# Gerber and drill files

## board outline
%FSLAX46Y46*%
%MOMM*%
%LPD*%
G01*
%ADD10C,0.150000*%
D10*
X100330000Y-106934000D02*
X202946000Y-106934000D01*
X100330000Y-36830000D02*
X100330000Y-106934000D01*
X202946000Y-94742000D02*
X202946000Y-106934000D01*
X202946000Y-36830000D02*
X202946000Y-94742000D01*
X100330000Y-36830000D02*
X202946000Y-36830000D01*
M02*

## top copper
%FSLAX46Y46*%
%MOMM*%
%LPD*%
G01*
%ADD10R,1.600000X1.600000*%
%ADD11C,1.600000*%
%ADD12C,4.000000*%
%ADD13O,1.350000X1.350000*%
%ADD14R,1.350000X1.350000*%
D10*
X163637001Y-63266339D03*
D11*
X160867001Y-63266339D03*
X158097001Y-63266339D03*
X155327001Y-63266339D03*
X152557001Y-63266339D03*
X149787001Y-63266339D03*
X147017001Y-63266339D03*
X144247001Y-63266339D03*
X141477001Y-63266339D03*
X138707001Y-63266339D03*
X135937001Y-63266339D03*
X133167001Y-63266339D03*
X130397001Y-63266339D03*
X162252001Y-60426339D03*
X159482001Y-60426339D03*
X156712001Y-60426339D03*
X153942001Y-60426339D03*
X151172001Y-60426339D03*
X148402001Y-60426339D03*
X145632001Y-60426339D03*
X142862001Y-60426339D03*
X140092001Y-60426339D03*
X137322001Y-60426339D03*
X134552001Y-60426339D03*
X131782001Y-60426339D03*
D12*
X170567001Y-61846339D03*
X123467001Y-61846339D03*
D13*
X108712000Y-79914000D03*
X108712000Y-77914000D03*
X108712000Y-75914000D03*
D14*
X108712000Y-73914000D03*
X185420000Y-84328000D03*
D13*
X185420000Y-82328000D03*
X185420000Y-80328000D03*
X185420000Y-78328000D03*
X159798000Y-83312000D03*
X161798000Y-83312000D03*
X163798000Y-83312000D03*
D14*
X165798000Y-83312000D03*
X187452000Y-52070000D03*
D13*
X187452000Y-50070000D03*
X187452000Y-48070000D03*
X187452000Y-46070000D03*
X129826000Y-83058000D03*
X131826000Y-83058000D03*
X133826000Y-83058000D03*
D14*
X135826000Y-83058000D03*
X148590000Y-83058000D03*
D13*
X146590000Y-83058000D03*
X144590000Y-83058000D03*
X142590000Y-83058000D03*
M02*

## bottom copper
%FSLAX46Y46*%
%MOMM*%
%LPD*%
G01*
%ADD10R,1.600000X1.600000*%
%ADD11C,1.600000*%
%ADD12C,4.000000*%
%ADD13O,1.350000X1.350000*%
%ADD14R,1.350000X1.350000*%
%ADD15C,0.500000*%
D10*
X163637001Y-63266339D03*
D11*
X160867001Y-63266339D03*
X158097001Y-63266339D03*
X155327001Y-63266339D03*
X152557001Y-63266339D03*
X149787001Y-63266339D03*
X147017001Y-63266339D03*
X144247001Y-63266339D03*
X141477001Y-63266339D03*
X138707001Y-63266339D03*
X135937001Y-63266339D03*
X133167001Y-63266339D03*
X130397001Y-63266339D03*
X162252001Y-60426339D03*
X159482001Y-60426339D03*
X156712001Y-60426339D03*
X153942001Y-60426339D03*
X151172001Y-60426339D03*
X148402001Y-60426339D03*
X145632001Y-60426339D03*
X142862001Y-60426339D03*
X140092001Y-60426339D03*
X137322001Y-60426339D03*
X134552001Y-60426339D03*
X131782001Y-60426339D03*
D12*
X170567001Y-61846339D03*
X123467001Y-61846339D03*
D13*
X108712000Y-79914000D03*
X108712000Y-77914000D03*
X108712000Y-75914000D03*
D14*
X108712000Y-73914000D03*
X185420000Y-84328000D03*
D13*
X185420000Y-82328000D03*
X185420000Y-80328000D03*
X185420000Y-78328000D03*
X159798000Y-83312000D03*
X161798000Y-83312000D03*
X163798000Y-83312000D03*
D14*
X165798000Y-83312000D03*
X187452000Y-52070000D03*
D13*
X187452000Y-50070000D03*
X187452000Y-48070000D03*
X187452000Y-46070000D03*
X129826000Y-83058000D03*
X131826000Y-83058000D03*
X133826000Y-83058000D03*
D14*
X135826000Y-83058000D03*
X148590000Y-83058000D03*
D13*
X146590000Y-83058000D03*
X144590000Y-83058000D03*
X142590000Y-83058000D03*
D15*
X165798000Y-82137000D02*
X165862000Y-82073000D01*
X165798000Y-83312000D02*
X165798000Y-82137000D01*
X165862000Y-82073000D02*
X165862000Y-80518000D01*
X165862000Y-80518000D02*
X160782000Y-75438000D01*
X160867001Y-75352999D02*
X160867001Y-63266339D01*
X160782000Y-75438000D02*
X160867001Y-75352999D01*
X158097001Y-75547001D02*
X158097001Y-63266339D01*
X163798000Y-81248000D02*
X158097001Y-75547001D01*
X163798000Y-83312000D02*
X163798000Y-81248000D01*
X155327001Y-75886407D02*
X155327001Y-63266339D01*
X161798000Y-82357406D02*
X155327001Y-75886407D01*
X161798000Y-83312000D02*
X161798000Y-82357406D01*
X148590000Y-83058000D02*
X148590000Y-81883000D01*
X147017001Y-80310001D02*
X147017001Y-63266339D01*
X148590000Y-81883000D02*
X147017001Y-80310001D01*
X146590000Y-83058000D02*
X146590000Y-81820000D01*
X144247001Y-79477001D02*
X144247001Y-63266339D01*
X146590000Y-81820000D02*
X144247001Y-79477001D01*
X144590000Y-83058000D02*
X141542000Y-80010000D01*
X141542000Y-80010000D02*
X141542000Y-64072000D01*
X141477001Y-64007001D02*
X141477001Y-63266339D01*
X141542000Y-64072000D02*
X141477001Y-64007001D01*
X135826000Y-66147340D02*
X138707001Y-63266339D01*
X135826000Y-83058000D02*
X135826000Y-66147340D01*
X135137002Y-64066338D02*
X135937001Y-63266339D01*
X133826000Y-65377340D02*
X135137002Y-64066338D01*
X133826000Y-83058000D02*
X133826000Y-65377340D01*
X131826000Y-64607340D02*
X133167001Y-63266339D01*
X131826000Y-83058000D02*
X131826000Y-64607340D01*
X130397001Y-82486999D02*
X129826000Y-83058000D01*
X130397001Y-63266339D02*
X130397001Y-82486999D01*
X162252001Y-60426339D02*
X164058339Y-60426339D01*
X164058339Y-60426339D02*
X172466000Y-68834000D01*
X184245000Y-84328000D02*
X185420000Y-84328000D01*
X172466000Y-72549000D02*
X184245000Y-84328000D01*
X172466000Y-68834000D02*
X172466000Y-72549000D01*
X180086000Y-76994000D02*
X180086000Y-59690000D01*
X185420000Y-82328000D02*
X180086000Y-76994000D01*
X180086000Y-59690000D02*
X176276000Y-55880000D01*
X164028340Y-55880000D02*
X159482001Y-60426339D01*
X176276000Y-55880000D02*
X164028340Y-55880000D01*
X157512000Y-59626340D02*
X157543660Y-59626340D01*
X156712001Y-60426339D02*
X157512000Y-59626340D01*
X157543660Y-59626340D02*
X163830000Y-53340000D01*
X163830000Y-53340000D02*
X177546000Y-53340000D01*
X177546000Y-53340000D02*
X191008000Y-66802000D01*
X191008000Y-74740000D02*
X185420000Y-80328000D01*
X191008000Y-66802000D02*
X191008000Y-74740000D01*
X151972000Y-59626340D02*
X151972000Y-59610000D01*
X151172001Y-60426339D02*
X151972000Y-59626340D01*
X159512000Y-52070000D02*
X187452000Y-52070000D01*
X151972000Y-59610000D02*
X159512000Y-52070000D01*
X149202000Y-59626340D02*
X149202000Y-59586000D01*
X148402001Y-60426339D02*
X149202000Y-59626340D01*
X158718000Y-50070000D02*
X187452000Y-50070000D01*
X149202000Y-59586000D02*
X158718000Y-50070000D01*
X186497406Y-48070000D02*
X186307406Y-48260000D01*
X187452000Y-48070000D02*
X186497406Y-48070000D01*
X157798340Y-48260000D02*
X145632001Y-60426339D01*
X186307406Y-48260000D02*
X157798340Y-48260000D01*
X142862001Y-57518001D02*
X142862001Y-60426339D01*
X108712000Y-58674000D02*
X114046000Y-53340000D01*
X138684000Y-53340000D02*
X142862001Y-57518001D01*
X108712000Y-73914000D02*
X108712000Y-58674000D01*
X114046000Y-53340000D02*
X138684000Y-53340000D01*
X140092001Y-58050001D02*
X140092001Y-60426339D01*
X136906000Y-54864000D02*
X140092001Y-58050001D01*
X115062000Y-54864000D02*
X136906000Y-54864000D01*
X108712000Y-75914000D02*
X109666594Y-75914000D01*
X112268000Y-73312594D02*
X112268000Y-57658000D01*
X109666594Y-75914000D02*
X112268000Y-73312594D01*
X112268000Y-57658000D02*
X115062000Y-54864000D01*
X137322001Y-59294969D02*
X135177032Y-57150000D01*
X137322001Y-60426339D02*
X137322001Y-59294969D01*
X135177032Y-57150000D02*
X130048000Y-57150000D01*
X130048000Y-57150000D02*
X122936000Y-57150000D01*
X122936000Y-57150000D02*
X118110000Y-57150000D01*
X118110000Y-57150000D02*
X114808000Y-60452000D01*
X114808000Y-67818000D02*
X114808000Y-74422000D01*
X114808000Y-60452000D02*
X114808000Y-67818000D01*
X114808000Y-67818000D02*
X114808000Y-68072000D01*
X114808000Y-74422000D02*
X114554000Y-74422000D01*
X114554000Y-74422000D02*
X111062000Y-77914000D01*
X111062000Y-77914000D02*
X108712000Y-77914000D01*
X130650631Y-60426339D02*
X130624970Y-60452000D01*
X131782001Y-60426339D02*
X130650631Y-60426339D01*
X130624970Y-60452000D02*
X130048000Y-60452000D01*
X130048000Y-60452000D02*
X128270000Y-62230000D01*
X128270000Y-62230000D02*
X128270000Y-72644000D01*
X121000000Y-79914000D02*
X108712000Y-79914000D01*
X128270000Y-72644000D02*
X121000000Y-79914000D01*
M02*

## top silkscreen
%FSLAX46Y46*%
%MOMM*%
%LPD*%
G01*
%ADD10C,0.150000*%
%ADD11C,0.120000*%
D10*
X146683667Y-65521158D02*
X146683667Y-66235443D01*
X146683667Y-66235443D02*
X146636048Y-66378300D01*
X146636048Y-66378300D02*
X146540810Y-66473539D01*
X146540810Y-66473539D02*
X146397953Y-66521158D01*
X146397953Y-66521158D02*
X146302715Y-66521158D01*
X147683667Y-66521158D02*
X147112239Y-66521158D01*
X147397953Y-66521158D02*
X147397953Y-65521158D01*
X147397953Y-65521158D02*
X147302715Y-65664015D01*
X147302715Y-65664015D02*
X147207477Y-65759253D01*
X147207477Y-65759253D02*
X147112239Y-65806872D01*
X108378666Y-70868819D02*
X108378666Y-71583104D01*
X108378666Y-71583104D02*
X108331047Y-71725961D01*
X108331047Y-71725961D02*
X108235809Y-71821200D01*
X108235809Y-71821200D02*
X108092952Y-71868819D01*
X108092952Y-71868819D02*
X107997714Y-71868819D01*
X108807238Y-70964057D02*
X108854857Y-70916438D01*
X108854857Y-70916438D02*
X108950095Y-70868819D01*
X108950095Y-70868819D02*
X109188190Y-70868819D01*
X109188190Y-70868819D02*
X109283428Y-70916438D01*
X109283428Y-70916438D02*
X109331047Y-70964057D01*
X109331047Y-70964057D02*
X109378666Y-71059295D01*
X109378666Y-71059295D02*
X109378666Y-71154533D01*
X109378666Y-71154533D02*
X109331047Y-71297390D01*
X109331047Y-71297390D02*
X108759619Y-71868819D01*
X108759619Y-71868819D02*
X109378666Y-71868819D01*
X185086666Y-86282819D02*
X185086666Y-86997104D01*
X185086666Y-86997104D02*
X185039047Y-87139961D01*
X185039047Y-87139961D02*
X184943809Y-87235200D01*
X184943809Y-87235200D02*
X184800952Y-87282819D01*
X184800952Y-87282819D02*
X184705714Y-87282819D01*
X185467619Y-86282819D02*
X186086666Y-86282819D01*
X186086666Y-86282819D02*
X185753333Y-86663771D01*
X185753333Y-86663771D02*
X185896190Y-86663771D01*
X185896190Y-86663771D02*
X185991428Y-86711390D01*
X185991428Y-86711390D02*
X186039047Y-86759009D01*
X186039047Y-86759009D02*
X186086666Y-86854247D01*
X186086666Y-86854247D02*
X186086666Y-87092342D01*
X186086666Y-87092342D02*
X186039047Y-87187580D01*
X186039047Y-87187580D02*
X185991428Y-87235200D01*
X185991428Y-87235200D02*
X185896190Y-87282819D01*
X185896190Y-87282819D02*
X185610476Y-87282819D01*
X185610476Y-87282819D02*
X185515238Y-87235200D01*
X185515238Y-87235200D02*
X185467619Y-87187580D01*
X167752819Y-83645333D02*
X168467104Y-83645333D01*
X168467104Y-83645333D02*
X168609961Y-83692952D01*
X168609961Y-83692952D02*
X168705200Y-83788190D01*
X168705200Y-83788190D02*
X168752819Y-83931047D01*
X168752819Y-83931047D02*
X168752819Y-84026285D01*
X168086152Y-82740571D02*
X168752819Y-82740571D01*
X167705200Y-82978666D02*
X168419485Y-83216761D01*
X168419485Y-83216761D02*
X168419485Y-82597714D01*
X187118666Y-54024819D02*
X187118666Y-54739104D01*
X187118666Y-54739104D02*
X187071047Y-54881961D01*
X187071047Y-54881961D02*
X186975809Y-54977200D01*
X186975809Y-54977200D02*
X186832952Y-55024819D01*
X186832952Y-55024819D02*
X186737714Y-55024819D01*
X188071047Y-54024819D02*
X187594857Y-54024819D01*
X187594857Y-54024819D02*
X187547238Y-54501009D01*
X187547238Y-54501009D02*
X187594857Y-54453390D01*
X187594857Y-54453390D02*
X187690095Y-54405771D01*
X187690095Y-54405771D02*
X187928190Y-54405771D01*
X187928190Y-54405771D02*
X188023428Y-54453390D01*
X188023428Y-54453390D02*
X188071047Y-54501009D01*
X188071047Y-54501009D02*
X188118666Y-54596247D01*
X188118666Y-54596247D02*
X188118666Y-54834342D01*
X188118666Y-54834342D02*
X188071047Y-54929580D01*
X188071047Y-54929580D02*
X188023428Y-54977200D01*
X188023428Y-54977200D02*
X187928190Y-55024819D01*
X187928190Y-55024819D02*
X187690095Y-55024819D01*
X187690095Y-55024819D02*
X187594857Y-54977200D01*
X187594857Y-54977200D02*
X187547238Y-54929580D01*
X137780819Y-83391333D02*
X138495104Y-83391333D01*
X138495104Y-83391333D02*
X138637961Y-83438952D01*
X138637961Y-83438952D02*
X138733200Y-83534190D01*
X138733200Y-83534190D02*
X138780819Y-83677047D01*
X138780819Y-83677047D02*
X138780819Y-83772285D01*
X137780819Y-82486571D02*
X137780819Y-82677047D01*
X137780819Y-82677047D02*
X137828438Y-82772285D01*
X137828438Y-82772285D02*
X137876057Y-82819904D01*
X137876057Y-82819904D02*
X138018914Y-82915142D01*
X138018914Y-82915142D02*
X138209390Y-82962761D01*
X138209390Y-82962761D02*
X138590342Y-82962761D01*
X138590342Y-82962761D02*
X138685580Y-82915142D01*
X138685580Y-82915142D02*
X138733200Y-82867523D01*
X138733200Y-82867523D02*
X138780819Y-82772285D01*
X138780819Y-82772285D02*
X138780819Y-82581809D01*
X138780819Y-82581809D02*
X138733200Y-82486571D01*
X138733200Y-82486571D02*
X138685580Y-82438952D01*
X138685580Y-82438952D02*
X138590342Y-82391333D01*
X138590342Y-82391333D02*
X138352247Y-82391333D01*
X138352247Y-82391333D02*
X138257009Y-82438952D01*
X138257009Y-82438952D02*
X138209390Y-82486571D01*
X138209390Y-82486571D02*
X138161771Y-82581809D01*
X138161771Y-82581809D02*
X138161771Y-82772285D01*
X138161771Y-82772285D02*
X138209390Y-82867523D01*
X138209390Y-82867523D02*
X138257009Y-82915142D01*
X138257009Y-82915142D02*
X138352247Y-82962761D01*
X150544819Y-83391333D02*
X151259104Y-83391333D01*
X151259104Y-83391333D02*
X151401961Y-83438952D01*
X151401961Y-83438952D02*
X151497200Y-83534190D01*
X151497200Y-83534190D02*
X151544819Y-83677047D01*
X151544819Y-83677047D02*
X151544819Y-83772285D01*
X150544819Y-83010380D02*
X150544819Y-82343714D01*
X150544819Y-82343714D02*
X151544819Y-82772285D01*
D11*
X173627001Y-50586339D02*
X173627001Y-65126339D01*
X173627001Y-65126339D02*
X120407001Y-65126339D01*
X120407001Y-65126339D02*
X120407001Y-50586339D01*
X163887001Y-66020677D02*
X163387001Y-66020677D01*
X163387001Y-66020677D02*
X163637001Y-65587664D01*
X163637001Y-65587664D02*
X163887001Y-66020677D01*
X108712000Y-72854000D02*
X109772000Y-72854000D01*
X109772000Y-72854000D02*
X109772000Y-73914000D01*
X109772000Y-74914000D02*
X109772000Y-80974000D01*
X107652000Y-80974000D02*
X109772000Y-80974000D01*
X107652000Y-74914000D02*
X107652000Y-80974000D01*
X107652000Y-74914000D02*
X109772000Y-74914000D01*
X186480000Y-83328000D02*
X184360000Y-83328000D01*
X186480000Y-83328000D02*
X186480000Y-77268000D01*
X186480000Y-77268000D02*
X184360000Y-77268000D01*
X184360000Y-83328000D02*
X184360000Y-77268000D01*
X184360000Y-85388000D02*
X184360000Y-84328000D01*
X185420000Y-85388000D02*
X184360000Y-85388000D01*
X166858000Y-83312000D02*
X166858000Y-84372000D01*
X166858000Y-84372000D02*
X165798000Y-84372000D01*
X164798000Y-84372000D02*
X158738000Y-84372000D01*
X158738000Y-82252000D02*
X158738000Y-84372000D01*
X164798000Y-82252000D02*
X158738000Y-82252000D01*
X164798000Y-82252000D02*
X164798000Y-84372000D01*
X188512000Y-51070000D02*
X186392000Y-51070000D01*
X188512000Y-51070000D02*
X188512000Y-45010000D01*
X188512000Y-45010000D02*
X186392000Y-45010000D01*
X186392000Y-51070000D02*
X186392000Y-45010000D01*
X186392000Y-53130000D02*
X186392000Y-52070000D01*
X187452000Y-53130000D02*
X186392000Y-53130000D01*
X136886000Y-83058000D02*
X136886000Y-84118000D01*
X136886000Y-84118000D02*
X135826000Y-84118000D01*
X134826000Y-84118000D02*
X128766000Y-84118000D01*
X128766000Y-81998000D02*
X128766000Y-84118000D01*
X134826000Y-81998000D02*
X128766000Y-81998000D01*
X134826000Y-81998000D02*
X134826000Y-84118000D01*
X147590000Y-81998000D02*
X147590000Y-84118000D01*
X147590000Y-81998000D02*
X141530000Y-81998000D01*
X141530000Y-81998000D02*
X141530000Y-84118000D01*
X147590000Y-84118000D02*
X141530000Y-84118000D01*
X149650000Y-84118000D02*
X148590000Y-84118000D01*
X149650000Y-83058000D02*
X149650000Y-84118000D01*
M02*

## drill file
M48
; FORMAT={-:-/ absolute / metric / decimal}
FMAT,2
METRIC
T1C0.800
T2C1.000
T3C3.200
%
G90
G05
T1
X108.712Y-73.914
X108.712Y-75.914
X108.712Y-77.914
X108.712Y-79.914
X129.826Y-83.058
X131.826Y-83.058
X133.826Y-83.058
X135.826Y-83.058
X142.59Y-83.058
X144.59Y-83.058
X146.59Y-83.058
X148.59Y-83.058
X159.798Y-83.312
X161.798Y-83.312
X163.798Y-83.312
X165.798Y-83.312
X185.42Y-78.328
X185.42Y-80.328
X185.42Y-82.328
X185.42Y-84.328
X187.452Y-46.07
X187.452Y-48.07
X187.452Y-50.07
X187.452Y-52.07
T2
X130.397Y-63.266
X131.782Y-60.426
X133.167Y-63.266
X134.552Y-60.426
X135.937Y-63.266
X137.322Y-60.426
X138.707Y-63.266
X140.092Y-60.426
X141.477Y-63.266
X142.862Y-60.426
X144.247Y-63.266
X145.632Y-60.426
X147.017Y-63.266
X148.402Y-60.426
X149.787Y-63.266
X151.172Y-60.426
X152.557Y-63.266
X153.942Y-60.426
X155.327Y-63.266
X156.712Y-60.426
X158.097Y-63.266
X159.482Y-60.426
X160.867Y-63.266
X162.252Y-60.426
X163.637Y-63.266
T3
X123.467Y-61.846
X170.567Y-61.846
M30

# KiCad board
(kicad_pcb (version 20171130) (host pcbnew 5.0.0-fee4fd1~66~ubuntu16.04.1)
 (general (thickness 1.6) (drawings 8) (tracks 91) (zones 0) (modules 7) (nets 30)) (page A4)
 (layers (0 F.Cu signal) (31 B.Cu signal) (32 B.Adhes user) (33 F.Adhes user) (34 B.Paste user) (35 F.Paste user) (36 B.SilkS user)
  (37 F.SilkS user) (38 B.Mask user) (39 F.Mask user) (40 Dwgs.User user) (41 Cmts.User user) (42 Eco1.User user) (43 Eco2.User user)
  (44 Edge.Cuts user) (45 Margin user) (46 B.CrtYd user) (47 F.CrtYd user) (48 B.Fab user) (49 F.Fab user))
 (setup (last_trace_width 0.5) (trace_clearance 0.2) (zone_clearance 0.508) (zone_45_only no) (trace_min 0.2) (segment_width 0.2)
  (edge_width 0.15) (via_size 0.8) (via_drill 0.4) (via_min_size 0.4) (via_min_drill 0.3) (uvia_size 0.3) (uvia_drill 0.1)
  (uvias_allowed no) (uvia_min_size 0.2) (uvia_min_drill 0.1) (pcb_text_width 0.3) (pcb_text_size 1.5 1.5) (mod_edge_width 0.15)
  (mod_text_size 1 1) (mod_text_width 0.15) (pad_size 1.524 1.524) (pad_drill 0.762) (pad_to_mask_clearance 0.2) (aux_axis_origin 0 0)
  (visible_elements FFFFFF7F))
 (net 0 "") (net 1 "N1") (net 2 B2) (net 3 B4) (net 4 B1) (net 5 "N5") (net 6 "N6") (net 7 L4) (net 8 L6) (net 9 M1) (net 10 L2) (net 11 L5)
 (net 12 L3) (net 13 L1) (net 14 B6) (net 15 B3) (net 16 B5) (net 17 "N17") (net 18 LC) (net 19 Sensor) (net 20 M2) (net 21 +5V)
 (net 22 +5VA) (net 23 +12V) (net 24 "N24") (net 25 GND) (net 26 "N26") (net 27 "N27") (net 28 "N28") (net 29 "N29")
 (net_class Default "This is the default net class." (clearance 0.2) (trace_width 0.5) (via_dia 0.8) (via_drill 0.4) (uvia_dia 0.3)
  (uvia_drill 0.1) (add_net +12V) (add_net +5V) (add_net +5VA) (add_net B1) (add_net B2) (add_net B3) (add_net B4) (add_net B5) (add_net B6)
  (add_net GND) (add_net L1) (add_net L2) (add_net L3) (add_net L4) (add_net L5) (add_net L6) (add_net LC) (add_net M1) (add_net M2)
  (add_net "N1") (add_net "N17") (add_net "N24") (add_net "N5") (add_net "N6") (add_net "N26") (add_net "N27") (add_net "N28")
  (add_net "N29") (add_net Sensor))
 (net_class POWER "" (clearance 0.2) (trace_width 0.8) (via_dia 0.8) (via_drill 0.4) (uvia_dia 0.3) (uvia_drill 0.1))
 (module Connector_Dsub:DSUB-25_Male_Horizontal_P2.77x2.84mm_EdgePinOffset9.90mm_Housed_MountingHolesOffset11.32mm (layer F.Cu)
  (at 163.637001 63.266339 180)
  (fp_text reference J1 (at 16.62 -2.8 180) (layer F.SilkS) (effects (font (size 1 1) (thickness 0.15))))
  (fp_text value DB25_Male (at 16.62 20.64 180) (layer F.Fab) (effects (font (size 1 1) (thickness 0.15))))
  (fp_line (start -9.99 12.68) (end -9.99 -1.86) (layer F.SilkS) (width 0.12))
  (fp_line (start -9.99 -1.86) (end 43.23 -1.86) (layer F.SilkS) (width 0.12))
  (fp_line (start 43.23 -1.86) (end 43.23 12.68) (layer F.SilkS) (width 0.12))
  (fp_line (start -0.25 -2.754338) (end 0.25 -2.754338) (layer F.SilkS) (width 0.12))
  (fp_line (start 0.25 -2.754338) (end 0 -2.321325) (layer F.SilkS) (width 0.12))
  (fp_line (start 0 -2.321325) (end -0.25 -2.754338) (layer F.SilkS) (width 0.12))
  (pad 1 thru_hole rect (at 0 0 180) (size 1.6 1.6) (drill 1) (layers *.Cu *.Mask) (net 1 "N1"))
  (pad 2 thru_hole circle (at 2.77 0 180) (size 1.6 1.6) (drill 1) (layers *.Cu *.Mask) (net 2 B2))
  (pad 3 thru_hole circle (at 5.54 0 180) (size 1.6 1.6) (drill 1) (layers *.Cu *.Mask) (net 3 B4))
  (pad 4 thru_hole circle (at 8.31 0 180) (size 1.6 1.6) (drill 1) (layers *.Cu *.Mask) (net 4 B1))
  (pad 5 thru_hole circle (at 11.08 0 180) (size 1.6 1.6) (drill 1) (layers *.Cu *.Mask) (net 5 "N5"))
  (pad 6 thru_hole circle (at 13.85 0 180) (size 1.6 1.6) (drill 1) (layers *.Cu *.Mask) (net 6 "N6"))
  (pad 7 thru_hole circle (at 16.62 0 180) (size 1.6 1.6) (drill 1) (layers *.Cu *.Mask) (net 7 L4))
  (pad 8 thru_hole circle (at 19.39 0 180) (size 1.6 1.6) (drill 1) (layers *.Cu *.Mask) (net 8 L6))
  (pad 9 thru_hole circle (at 22.16 0 180) (size 1.6 1.6) (drill 1) (layers *.Cu *.Mask) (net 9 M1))
  (pad 10 thru_hole circle (at 24.93 0 180) (size 1.6 1.6) (drill 1) (layers *.Cu *.Mask) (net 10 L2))
  (pad 11 thru_hole circle (at 27.7 0 180) (size 1.6 1.6) (drill 1) (layers *.Cu *.Mask) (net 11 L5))
  (pad 12 thru_hole circle (at 30.47 0 180) (size 1.6 1.6) (drill 1) (layers *.Cu *.Mask) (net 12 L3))
  (pad 13 thru_hole circle (at 33.24 0 180) (size 1.6 1.6) (drill 1) (layers *.Cu *.Mask) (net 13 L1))
  (pad 14 thru_hole circle (at 1.385 2.84 180) (size 1.6 1.6) (drill 1) (layers *.Cu *.Mask) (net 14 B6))
  (pad 15 thru_hole circle (at 4.155 2.84 180) (size 1.6 1.6) (drill 1) (layers *.Cu *.Mask) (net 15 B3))
  (pad 16 thru_hole circle (at 6.925 2.84 180) (size 1.6 1.6) (drill 1) (layers *.Cu *.Mask) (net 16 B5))
  (pad 17 thru_hole circle (at 9.695 2.84 180) (size 1.6 1.6) (drill 1) (layers *.Cu *.Mask) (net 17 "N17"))
  (pad 18 thru_hole circle (at 12.465 2.84 180) (size 1.6 1.6) (drill 1) (layers *.Cu *.Mask) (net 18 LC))
  (pad 19 thru_hole circle (at 15.235 2.84 180) (size 1.6 1.6) (drill 1) (layers *.Cu *.Mask) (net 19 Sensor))
  (pad 20 thru_hole circle (at 18.005 2.84 180) (size 1.6 1.6) (drill 1) (layers *.Cu *.Mask) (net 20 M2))
  (pad 21 thru_hole circle (at 20.775 2.84 180) (size 1.6 1.6) (drill 1) (layers *.Cu *.Mask) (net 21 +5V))
  (pad 22 thru_hole circle (at 23.545 2.84 180) (size 1.6 1.6) (drill 1) (layers *.Cu *.Mask) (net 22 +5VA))
  (pad 23 thru_hole circle (at 26.315 2.84 180) (size 1.6 1.6) (drill 1) (layers *.Cu *.Mask) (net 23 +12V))
  (pad 24 thru_hole circle (at 29.085 2.84 180) (size 1.6 1.6) (drill 1) (layers *.Cu *.Mask) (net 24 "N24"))
  (pad 25 thru_hole circle (at 31.855 2.84 180) (size 1.6 1.6) (drill 1) (layers *.Cu *.Mask) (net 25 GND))
  (pad 0 thru_hole circle (at -6.93 1.42 180) (size 4 4) (drill 3.2) (layers *.Cu *.Mask))
  (pad 0 thru_hole circle (at 40.17 1.42 180) (size 4 4) (drill 3.2) (layers *.Cu *.Mask)))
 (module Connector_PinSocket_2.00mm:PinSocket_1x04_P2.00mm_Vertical (layer F.Cu) (at 108.712 73.914)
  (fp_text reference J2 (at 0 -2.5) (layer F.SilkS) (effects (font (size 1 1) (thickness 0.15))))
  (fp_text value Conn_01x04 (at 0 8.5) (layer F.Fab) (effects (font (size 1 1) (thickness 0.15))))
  (fp_line (start 0 -1.06) (end 1.06 -1.06) (layer F.SilkS) (width 0.12))
  (fp_line (start 1.06 -1.06) (end 1.06 0) (layer F.SilkS) (width 0.12))
  (fp_line (start 1.06 1) (end 1.06 7.06) (layer F.SilkS) (width 0.12))
  (fp_line (start -1.06 7.06) (end 1.06 7.06) (layer F.SilkS) (width 0.12))
  (fp_line (start -1.06 1) (end -1.06 7.06) (layer F.SilkS) (width 0.12))
  (fp_line (start -1.06 1) (end 1.06 1) (layer F.SilkS) (width 0.12))
  (pad 4 thru_hole oval (at 0 6) (size 1.35 1.35) (drill 0.8) (layers *.Cu *.Mask) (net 25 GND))
  (pad 3 thru_hole oval (at 0 4) (size 1.35 1.35) (drill 0.8) (layers *.Cu *.Mask) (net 23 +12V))
  (pad 2 thru_hole oval (at 0 2) (size 1.35 1.35) (drill 0.8) (layers *.Cu *.Mask) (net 22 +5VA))
  (pad 1 thru_hole rect (at 0 0) (size 1.35 1.35) (drill 0.8) (layers *.Cu *.Mask) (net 21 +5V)))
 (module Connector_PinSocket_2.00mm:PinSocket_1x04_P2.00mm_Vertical (layer F.Cu) (at 185.42 84.328 180)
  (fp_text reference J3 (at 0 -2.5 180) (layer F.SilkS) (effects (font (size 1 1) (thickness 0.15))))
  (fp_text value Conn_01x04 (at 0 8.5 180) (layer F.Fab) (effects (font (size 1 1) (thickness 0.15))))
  (fp_line (start -1.06 1) (end 1.06 1) (layer F.SilkS) (width 0.12))
  (fp_line (start -1.06 1) (end -1.06 7.06) (layer F.SilkS) (width 0.12))
  (fp_line (start -1.06 7.06) (end 1.06 7.06) (layer F.SilkS) (width 0.12))
  (fp_line (start 1.06 1) (end 1.06 7.06) (layer F.SilkS) (width 0.12))
  (fp_line (start 1.06 -1.06) (end 1.06 0) (layer F.SilkS) (width 0.12))
  (fp_line (start 0 -1.06) (end 1.06 -1.06) (layer F.SilkS) (width 0.12))
  (pad 1 thru_hole rect (at 0 0 180) (size 1.35 1.35) (drill 0.8) (layers *.Cu *.Mask) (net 14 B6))
  (pad 2 thru_hole oval (at 0 2 180) (size 1.35 1.35) (drill 0.8) (layers *.Cu *.Mask) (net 15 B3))
  (pad 3 thru_hole oval (at 0 4 180) (size 1.35 1.35) (drill 0.8) (layers *.Cu *.Mask) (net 16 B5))
  (pad 4 thru_hole oval (at 0 6 180) (size 1.35 1.35) (drill 0.8) (layers *.Cu *.Mask) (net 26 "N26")))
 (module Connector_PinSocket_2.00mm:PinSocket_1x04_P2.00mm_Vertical (layer F.Cu) (at 165.798 83.312 270)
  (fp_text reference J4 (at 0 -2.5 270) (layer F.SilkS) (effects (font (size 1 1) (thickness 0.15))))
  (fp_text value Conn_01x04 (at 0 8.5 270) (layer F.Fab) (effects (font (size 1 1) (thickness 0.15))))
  (fp_line (start 0 -1.06) (end 1.06 -1.06) (layer F.SilkS) (width 0.12))
  (fp_line (start 1.06 -1.06) (end 1.06 0) (layer F.SilkS) (width 0.12))
  (fp_line (start 1.06 1) (end 1.06 7.06) (layer F.SilkS) (width 0.12))
  (fp_line (start -1.06 7.06) (end 1.06 7.06) (layer F.SilkS) (width 0.12))
  (fp_line (start -1.06 1) (end -1.06 7.06) (layer F.SilkS) (width 0.12))
  (fp_line (start -1.06 1) (end 1.06 1) (layer F.SilkS) (width 0.12))
  (pad 4 thru_hole oval (at 0 6 270) (size 1.35 1.35) (drill 0.8) (layers *.Cu *.Mask) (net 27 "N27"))
  (pad 3 thru_hole oval (at 0 4 270) (size 1.35 1.35) (drill 0.8) (layers *.Cu *.Mask) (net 4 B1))
  (pad 2 thru_hole oval (at 0 2 270) (size 1.35 1.35) (drill 0.8) (layers *.Cu *.Mask) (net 3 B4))
  (pad 1 thru_hole rect (at 0 0 270) (size 1.35 1.35) (drill 0.8) (layers *.Cu *.Mask) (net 2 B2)))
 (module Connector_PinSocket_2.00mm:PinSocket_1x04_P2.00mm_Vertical (layer F.Cu) (at 187.452 52.07 180)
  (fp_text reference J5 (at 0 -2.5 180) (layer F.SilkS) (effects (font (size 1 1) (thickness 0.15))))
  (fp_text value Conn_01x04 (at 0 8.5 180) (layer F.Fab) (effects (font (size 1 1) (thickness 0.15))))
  (fp_line (start -1.06 1) (end 1.06 1) (layer F.SilkS) (width 0.12))
  (fp_line (start -1.06 1) (end -1.06 7.06) (layer F.SilkS) (width 0.12))
  (fp_line (start -1.06 7.06) (end 1.06 7.06) (layer F.SilkS) (width 0.12))
  (fp_line (start 1.06 1) (end 1.06 7.06) (layer F.SilkS) (width 0.12))
  (fp_line (start 1.06 -1.06) (end 1.06 0) (layer F.SilkS) (width 0.12))
  (fp_line (start 0 -1.06) (end 1.06 -1.06) (layer F.SilkS) (width 0.12))
  (pad 1 thru_hole rect (at 0 0 180) (size 1.35 1.35) (drill 0.8) (layers *.Cu *.Mask) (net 18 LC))
  (pad 2 thru_hole oval (at 0 2 180) (size 1.35 1.35) (drill 0.8) (layers *.Cu *.Mask) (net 19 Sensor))
  (pad 3 thru_hole oval (at 0 4 180) (size 1.35 1.35) (drill 0.8) (layers *.Cu *.Mask) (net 20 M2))
  (pad 4 thru_hole oval (at 0 6 180) (size 1.35 1.35) (drill 0.8) (layers *.Cu *.Mask) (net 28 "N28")))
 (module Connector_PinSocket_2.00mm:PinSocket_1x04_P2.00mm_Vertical (layer F.Cu) (at 135.826 83.058 270)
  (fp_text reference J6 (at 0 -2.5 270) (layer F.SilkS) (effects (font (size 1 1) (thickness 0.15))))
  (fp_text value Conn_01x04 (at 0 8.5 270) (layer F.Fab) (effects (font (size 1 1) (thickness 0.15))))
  (fp_line (start 0 -1.06) (end 1.06 -1.06) (layer F.SilkS) (width 0.12))
  (fp_line (start 1.06 -1.06) (end 1.06 0) (layer F.SilkS) (width 0.12))
  (fp_line (start 1.06 1) (end 1.06 7.06) (layer F.SilkS) (width 0.12))
  (fp_line (start -1.06 7.06) (end 1.06 7.06) (layer F.SilkS) (width 0.12))
  (fp_line (start -1.06 1) (end -1.06 7.06) (layer F.SilkS) (width 0.12))
  (fp_line (start -1.06 1) (end 1.06 1) (layer F.SilkS) (width 0.12))
  (pad 4 thru_hole oval (at 0 6 270) (size 1.35 1.35) (drill 0.8) (layers *.Cu *.Mask) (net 13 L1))
  (pad 3 thru_hole oval (at 0 4 270) (size 1.35 1.35) (drill 0.8) (layers *.Cu *.Mask) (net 12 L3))
  (pad 2 thru_hole oval (at 0 2 270) (size 1.35 1.35) (drill 0.8) (layers *.Cu *.Mask) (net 11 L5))
  (pad 1 thru_hole rect (at 0 0 270) (size 1.35 1.35) (drill 0.8) (layers *.Cu *.Mask) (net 10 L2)))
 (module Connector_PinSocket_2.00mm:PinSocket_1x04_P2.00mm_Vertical (layer F.Cu) (at 148.59 83.058 270)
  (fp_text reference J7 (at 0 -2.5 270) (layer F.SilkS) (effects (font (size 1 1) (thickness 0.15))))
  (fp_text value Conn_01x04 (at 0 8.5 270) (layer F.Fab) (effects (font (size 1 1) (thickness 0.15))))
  (fp_line (start -1.06 1) (end 1.06 1) (layer F.SilkS) (width 0.12))
  (fp_line (start -1.06 1) (end -1.06 7.06) (layer F.SilkS) (width 0.12))
  (fp_line (start -1.06 7.06) (end 1.06 7.06) (layer F.SilkS) (width 0.12))
  (fp_line (start 1.06 1) (end 1.06 7.06) (layer F.SilkS) (width 0.12))
  (fp_line (start 1.06 -1.06) (end 1.06 0) (layer F.SilkS) (width 0.12))
  (fp_line (start 0 -1.06) (end 1.06 -1.06) (layer F.SilkS) (width 0.12))
  (pad 1 thru_hole rect (at 0 0 270) (size 1.35 1.35) (drill 0.8) (layers *.Cu *.Mask) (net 7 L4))
  (pad 2 thru_hole oval (at 0 2 270) (size 1.35 1.35) (drill 0.8) (layers *.Cu *.Mask) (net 8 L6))
  (pad 3 thru_hole oval (at 0 4 270) (size 1.35 1.35) (drill 0.8) (layers *.Cu *.Mask) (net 9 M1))
  (pad 4 thru_hole oval (at 0 6 270) (size 1.35 1.35) (drill 0.8) (layers *.Cu *.Mask) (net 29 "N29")))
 (gr_line (start 100.33 106.934) (end 202.946 106.934) (layer Edge.Cuts) (width 0.15))
 (gr_line (start 100.33 36.83) (end 100.33 106.934) (layer Edge.Cuts) (width 0.15))
 (gr_line (start 202.946 94.742) (end 202.946 106.934) (layer Edge.Cuts) (width 0.15))
 (gr_line (start 202.946 36.83) (end 202.946 94.742) (layer Edge.Cuts) (width 0.15))
 (gr_line (start 100.33 36.83) (end 202.946 36.83) (layer Edge.Cuts) (width 0.15))
 (segment (start 165.798 82.137) (end 165.862 82.073) (width 0.5) (layer B.Cu) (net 2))
 (segment (start 165.798 83.312) (end 165.798 82.137) (width 0.5) (layer B.Cu) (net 2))
 (segment (start 165.862 82.073) (end 165.862 80.518) (width 0.5) (layer B.Cu) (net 2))
 (segment (start 165.862 80.518) (end 160.782 75.438) (width 0.5) (layer B.Cu) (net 2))
 (segment (start 160.867001 75.352999) (end 160.867001 63.266339) (width 0.5) (layer B.Cu) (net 2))
 (segment (start 160.782 75.438) (end 160.867001 75.352999) (width 0.5) (layer B.Cu) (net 2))
 (segment (start 158.097001 75.547001) (end 158.097001 63.266339) (width 0.5) (layer B.Cu) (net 3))
 (segment (start 163.798 81.248) (end 158.097001 75.547001) (width 0.5) (layer B.Cu) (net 3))
 (segment (start 163.798 83.312) (end 163.798 81.248) (width 0.5) (layer B.Cu) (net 3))
 (segment (start 155.327001 75.886407) (end 155.327001 63.266339) (width 0.5) (layer B.Cu) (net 4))
 (segment (start 161.798 82.357406) (end 155.327001 75.886407) (width 0.5) (layer B.Cu) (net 4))
 (segment (start 161.798 83.312) (end 161.798 82.357406) (width 0.5) (layer B.Cu) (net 4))
 (segment (start 148.59 83.058) (end 148.59 81.883) (width 0.5) (layer B.Cu) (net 7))
 (segment (start 147.017001 80.310001) (end 147.017001 63.266339) (width 0.5) (layer B.Cu) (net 7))
 (segment (start 148.59 81.883) (end 147.017001 80.310001) (width 0.5) (layer B.Cu) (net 7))
 (segment (start 146.59 83.058) (end 146.59 81.82) (width 0.5) (layer B.Cu) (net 8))
 (segment (start 144.247001 79.477001) (end 144.247001 63.266339) (width 0.5) (layer B.Cu) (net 8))
 (segment (start 146.59 81.82) (end 144.247001 79.477001) (width 0.5) (layer B.Cu) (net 8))
 (segment (start 144.59 83.058) (end 141.542 80.01) (width 0.5) (layer B.Cu) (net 9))
 (segment (start 141.542 80.01) (end 141.542 64.072) (width 0.5) (layer B.Cu) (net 9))
 (segment (start 141.477001 64.007001) (end 141.477001 63.266339) (width 0.5) (layer B.Cu) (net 9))
 (segment (start 141.542 64.072) (end 141.477001 64.007001) (width 0.5) (layer B.Cu) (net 9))
 (segment (start 135.826 66.14734) (end 138.707001 63.266339) (width 0.5) (layer B.Cu) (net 10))
 (segment (start 135.826 83.058) (end 135.826 66.14734) (width 0.5) (layer B.Cu) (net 10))
 (segment (start 135.137002 64.066338) (end 135.937001 63.266339) (width 0.5) (layer B.Cu) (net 11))
 (segment (start 133.826 65.37734) (end 135.137002 64.066338) (width 0.5) (layer B.Cu) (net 11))
 (segment (start 133.826 83.058) (end 133.826 65.37734) (width 0.5) (layer B.Cu) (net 11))
 (segment (start 131.826 64.60734) (end 133.167001 63.266339) (width 0.5) (layer B.Cu) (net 12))
 (segment (start 131.826 83.058) (end 131.826 64.60734) (width 0.5) (layer B.Cu) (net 12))
 (segment (start 130.397001 82.486999) (end 129.826 83.058) (width 0.5) (layer B.Cu) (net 13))
 (segment (start 130.397001 63.266339) (end 130.397001 82.486999) (width 0.5) (layer B.Cu) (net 13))
 (segment (start 162.252001 60.426339) (end 164.058339 60.426339) (width 0.5) (layer B.Cu) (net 14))
 (segment (start 164.058339 60.426339) (end 172.466 68.834) (width 0.5) (layer B.Cu) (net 14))
 (segment (start 184.245 84.328) (end 185.42 84.328) (width 0.5) (layer B.Cu) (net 14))
 (segment (start 172.466 72.549) (end 184.245 84.328) (width 0.5) (layer B.Cu) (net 14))
 (segment (start 172.466 68.834) (end 172.466 72.549) (width 0.5) (layer B.Cu) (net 14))
 (segment (start 180.086 76.994) (end 180.086 59.69) (width 0.5) (layer B.Cu) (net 15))
 (segment (start 185.42 82.328) (end 180.086 76.994) (width 0.5) (layer B.Cu) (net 15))
 (segment (start 180.086 59.69) (end 176.276 55.88) (width 0.5) (layer B.Cu) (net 15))
 (segment (start 164.02834 55.88) (end 159.482001 60.426339) (width 0.5) (layer B.Cu) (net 15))
 (segment (start 176.276 55.88) (end 164.02834 55.88) (width 0.5) (layer B.Cu) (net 15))
 (segment (start 157.512 59.62634) (end 157.54366 59.62634) (width 0.5) (layer B.Cu) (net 16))
 (segment (start 156.712001 60.426339) (end 157.512 59.62634) (width 0.5) (layer B.Cu) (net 16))
 (segment (start 157.54366 59.62634) (end 163.83 53.34) (width 0.5) (layer B.Cu) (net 16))
 (segment (start 163.83 53.34) (end 177.546 53.34) (width 0.5) (layer B.Cu) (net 16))
 (segment (start 177.546 53.34) (end 191.008 66.802) (width 0.5) (layer B.Cu) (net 16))
 (segment (start 191.008 74.74) (end 185.42 80.328) (width 0.5) (layer B.Cu) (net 16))
 (segment (start 191.008 66.802) (end 191.008 74.74) (width 0.5) (layer B.Cu) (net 16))
 (segment (start 151.972 59.62634) (end 151.972 59.61) (width 0.5) (layer B.Cu) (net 18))
 (segment (start 151.172001 60.426339) (end 151.972 59.62634) (width 0.5) (layer B.Cu) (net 18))
 (segment (start 159.512 52.07) (end 187.452 52.07) (width 0.5) (layer B.Cu) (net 18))
 (segment (start 151.972 59.61) (end 159.512 52.07) (width 0.5) (layer B.Cu) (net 18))
 (segment (start 149.202 59.62634) (end 149.202 59.586) (width 0.5) (layer B.Cu) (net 19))
 (segment (start 148.402001 60.426339) (end 149.202 59.62634) (width 0.5) (layer B.Cu) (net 19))
 (segment (start 158.718 50.07) (end 187.452 50.07) (width 0.5) (layer B.Cu) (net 19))
 (segment (start 149.202 59.586) (end 158.718 50.07) (width 0.5) (layer B.Cu) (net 19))
 (segment (start 186.497406 48.07) (end 186.307406 48.26) (width 0.5) (layer B.Cu) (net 20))
 (segment (start 187.452 48.07) (end 186.497406 48.07) (width 0.5) (layer B.Cu) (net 20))
 (segment (start 157.79834 48.26) (end 145.632001 60.426339) (width 0.5) (layer B.Cu) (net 20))
 (segment (start 186.307406 48.26) (end 157.79834 48.26) (width 0.5) (layer B.Cu) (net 20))
 (segment (start 142.862001 57.518001) (end 142.862001 60.426339) (width 0.5) (layer B.Cu) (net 21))
 (segment (start 108.712 58.674) (end 114.046 53.34) (width 0.5) (layer B.Cu) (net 21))
 (segment (start 138.684 53.34) (end 142.862001 57.518001) (width 0.5) (layer B.Cu) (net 21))
 (segment (start 108.712 73.914) (end 108.712 58.674) (width 0.5) (layer B.Cu) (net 21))
 (segment (start 114.046 53.34) (end 138.684 53.34) (width 0.5) (layer B.Cu) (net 21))
 (segment (start 140.092001 58.050001) (end 140.092001 60.426339) (width 0.5) (layer B.Cu) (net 22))
 (segment (start 136.906 54.864) (end 140.092001 58.050001) (width 0.5) (layer B.Cu) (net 22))
 (segment (start 115.062 54.864) (end 136.906 54.864) (width 0.5) (layer B.Cu) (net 22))
 (segment (start 108.712 75.914) (end 109.666594 75.914) (width 0.5) (layer B.Cu) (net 22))
 (segment (start 112.268 73.312594) (end 112.268 57.658) (width 0.5) (layer B.Cu) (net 22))
 (segment (start 109.666594 75.914) (end 112.268 73.312594) (width 0.5) (layer B.Cu) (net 22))
 (segment (start 112.268 57.658) (end 115.062 54.864) (width 0.5) (layer B.Cu) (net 22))
 (segment (start 137.322001 59.294969) (end 135.177032 57.15) (width 0.5) (layer B.Cu) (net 23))
 (segment (start 137.322001 60.426339) (end 137.322001 59.294969) (width 0.5) (layer B.Cu) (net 23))
 (segment (start 135.177032 57.15) (end 130.048 57.15) (width 0.5) (layer B.Cu) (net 23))
 (segment (start 130.048 57.15) (end 122.936 57.15) (width 0.5) (layer B.Cu) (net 23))
 (segment (start 122.936 57.15) (end 118.11 57.15) (width 0.5) (layer B.Cu) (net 23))
 (segment (start 118.11 57.15) (end 114.808 60.452) (width 0.5) (layer B.Cu) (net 23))
 (segment (start 114.808 67.818) (end 114.808 74.422) (width 0.5) (layer B.Cu) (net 23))
 (segment (start 114.808 60.452) (end 114.808 67.818) (width 0.5) (layer B.Cu) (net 23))
 (segment (start 114.808 67.818) (end 114.808 68.072) (width 0.5) (layer B.Cu) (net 23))
 (segment (start 114.808 74.422) (end 114.554 74.422) (width 0.5) (layer B.Cu) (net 23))
 (segment (start 114.554 74.422) (end 111.062 77.914) (width 0.5) (layer B.Cu) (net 23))
 (segment (start 111.062 77.914) (end 108.712 77.914) (width 0.5) (layer B.Cu) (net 23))
 (segment (start 130.650631 60.426339) (end 130.62497 60.452) (width 0.5) (layer B.Cu) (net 25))
 (segment (start 131.782001 60.426339) (end 130.650631 60.426339) (width 0.5) (layer B.Cu) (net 25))
 (segment (start 130.62497 60.452) (end 130.048 60.452) (width 0.5) (layer B.Cu) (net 25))
 (segment (start 130.048 60.452) (end 128.27 62.23) (width 0.5) (layer B.Cu) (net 25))
 (segment (start 128.27 62.23) (end 128.27 72.644) (width 0.5) (layer B.Cu) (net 25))
 (segment (start 121 79.914) (end 108.712 79.914) (width 0.5) (layer B.Cu) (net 25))
 (segment (start 128.27 72.644) (end 121 79.914) (width 0.5) (layer B.Cu) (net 25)))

